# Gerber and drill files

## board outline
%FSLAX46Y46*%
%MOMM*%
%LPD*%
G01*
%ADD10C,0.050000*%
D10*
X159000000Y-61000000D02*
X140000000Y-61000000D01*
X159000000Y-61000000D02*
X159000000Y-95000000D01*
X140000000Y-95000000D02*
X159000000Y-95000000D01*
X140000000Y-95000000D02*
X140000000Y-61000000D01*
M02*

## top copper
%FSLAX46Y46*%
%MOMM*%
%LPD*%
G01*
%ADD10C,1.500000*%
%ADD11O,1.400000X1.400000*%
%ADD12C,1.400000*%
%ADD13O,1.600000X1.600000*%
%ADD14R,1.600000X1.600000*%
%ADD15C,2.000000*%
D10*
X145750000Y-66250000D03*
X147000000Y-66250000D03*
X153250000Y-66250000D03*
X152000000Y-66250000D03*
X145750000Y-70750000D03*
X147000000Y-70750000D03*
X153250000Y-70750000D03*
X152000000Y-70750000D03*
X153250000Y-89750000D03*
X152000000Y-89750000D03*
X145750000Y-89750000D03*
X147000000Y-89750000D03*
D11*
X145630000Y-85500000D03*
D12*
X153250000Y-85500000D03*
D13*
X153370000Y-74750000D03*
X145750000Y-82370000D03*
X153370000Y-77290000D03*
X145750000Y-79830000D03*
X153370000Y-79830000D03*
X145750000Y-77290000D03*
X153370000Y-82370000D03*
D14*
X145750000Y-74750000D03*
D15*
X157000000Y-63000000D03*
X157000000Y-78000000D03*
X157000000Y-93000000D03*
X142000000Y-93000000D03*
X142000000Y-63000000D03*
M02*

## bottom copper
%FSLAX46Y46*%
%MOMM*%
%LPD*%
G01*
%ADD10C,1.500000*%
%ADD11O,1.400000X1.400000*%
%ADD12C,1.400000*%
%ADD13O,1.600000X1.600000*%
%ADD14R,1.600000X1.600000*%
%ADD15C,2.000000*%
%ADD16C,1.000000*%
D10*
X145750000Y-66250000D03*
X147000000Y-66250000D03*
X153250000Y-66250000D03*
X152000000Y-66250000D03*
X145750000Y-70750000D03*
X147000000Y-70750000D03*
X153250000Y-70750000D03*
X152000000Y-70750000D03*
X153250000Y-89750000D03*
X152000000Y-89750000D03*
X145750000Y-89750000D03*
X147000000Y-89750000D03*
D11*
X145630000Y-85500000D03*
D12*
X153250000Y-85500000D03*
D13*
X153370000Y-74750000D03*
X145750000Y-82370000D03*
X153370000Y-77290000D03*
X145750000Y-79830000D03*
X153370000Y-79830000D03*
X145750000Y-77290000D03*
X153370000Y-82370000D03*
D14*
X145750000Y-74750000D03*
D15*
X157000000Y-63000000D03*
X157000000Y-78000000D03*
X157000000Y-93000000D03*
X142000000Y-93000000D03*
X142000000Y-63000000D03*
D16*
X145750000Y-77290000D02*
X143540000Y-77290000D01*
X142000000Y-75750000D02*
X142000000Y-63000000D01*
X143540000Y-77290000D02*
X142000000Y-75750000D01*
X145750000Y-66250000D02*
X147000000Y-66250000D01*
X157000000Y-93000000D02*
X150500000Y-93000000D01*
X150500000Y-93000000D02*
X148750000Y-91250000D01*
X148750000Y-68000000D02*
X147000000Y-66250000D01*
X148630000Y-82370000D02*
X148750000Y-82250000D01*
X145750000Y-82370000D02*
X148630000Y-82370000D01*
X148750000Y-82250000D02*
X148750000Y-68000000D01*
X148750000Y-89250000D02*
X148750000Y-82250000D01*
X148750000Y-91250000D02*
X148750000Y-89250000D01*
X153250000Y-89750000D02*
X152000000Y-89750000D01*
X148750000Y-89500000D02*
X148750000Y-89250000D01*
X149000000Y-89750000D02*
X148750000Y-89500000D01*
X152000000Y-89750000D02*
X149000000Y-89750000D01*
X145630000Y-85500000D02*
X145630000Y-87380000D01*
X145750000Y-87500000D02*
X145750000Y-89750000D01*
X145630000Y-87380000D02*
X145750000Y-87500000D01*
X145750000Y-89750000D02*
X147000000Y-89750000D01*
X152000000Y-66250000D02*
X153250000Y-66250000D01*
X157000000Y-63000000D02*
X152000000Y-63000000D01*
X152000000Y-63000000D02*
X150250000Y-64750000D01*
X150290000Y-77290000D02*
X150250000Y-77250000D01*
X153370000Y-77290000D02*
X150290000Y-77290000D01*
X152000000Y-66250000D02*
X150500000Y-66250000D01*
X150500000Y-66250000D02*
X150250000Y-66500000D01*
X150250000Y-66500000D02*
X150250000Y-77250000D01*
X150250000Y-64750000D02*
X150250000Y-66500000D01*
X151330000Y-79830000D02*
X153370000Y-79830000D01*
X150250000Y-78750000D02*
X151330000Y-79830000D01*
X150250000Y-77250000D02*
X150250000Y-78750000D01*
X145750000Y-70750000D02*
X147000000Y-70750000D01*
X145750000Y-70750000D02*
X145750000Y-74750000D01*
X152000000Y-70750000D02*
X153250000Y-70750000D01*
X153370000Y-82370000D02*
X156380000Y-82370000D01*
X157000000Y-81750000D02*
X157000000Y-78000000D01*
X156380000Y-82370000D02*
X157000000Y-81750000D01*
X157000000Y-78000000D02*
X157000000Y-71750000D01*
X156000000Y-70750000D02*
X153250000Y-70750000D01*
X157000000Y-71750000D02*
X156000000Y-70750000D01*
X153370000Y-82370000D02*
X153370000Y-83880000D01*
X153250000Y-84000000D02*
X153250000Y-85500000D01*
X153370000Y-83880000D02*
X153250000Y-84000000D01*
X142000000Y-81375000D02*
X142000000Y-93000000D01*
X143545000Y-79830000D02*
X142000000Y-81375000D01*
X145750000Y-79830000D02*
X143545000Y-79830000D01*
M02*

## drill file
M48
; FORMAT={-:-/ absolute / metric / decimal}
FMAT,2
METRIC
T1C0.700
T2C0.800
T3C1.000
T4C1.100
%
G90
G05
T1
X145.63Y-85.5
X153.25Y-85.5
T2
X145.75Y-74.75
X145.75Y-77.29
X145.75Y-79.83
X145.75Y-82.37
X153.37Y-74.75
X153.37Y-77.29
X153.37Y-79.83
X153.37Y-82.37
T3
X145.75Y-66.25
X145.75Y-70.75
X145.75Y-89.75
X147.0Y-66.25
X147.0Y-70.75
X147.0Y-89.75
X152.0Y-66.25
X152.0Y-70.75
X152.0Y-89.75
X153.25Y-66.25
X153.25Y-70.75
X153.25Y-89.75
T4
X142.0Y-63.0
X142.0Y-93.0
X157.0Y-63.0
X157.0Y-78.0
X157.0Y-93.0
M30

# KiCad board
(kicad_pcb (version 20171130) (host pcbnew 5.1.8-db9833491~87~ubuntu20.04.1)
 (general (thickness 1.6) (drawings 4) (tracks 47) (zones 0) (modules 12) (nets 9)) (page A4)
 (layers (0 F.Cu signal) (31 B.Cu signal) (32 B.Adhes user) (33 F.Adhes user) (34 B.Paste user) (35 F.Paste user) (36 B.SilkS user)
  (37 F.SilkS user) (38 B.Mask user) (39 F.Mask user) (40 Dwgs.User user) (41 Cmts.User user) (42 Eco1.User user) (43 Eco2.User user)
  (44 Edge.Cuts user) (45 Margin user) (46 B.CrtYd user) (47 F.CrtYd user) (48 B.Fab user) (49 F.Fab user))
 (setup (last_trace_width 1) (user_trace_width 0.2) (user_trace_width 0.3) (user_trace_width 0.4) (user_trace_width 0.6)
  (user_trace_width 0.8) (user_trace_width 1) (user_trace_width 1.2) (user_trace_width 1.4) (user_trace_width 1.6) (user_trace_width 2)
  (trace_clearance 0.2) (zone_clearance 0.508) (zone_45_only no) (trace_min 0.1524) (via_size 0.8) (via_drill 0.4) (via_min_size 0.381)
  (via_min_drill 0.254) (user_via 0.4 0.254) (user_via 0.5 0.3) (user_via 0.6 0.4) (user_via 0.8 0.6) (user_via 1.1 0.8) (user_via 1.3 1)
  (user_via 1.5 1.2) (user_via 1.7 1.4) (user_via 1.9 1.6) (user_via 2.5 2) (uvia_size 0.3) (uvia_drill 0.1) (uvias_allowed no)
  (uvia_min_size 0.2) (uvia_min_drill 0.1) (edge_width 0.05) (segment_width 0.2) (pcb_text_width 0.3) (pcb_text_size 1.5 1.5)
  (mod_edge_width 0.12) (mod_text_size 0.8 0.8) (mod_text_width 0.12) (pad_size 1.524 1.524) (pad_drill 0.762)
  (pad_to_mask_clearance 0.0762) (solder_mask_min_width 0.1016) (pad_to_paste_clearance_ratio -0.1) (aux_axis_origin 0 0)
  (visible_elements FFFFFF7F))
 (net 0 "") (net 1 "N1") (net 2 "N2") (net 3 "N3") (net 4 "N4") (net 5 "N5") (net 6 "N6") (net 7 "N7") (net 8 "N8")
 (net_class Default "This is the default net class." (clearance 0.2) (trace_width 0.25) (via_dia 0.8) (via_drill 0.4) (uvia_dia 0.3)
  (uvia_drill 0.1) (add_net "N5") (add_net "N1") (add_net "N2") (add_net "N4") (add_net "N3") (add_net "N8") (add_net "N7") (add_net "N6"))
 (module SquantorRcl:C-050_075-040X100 (layer F.Cu) (at 149.5 66.25 180)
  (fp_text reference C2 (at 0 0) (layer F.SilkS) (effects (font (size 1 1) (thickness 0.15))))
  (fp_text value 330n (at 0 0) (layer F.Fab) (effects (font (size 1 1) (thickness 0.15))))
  (pad 2 thru_hole circle (at 3.75 0 180) (size 1.5 1.5) (drill 1) (layers *.Cu *.Mask) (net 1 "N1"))
  (pad 2 thru_hole circle (at 2.5 0 180) (size 1.5 1.5) (drill 1) (layers *.Cu *.Mask) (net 1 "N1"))
  (pad 1 thru_hole circle (at -3.75 0 180) (size 1.5 1.5) (drill 1) (layers *.Cu *.Mask) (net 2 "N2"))
  (pad 1 thru_hole circle (at -2.5 0 180) (size 1.5 1.5) (drill 1) (layers *.Cu *.Mask) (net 2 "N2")))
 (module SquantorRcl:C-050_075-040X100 (layer F.Cu) (at 149.5 70.75 180)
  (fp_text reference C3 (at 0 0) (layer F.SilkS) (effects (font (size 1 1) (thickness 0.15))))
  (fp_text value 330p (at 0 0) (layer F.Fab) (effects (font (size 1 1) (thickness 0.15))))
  (pad 2 thru_hole circle (at 3.75 0 180) (size 1.5 1.5) (drill 1) (layers *.Cu *.Mask) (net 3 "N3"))
  (pad 2 thru_hole circle (at 2.5 0 180) (size 1.5 1.5) (drill 1) (layers *.Cu *.Mask) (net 3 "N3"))
  (pad 1 thru_hole circle (at -3.75 0 180) (size 1.5 1.5) (drill 1) (layers *.Cu *.Mask) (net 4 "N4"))
  (pad 1 thru_hole circle (at -2.5 0 180) (size 1.5 1.5) (drill 1) (layers *.Cu *.Mask) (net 4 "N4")))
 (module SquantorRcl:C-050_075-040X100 (layer F.Cu) (at 149.5 89.75)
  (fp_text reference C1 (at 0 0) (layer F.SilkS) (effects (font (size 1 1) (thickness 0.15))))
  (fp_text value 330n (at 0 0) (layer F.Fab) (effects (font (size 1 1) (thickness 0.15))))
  (pad 2 thru_hole circle (at 3.75 0) (size 1.5 1.5) (drill 1) (layers *.Cu *.Mask) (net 1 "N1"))
  (pad 2 thru_hole circle (at 2.5 0) (size 1.5 1.5) (drill 1) (layers *.Cu *.Mask) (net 1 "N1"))
  (pad 1 thru_hole circle (at -3.75 0) (size 1.5 1.5) (drill 1) (layers *.Cu *.Mask) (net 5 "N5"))
  (pad 1 thru_hole circle (at -2.5 0) (size 1.5 1.5) (drill 1) (layers *.Cu *.Mask) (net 5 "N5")))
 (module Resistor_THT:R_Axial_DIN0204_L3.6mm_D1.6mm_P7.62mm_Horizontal (layer F.Cu) (at 153.25 85.5 180)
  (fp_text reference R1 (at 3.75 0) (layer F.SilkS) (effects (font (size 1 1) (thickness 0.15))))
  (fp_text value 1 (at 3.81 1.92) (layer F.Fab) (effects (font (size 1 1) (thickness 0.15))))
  (pad 2 thru_hole oval (at 7.62 0 180) (size 1.4 1.4) (drill 0.7) (layers *.Cu *.Mask) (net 5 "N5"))
  (pad 1 thru_hole circle (at 0 0 180) (size 1.4 1.4) (drill 0.7) (layers *.Cu *.Mask) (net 4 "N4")))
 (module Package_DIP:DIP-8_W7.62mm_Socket (layer F.Cu) (at 145.75 74.75)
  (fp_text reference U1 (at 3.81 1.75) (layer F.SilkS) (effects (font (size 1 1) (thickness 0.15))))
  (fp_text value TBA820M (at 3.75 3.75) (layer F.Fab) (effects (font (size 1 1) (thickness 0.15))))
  (pad 8 thru_hole oval (at 7.62 0) (size 1.6 1.6) (drill 0.8) (layers *.Cu *.Mask) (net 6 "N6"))
  (pad 4 thru_hole oval (at 0 7.62) (size 1.6 1.6) (drill 0.8) (layers *.Cu *.Mask) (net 1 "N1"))
  (pad 7 thru_hole oval (at 7.62 2.54) (size 1.6 1.6) (drill 0.8) (layers *.Cu *.Mask) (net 2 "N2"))
  (pad 3 thru_hole oval (at 0 5.08) (size 1.6 1.6) (drill 0.8) (layers *.Cu *.Mask) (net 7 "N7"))
  (pad 6 thru_hole oval (at 7.62 5.08) (size 1.6 1.6) (drill 0.8) (layers *.Cu *.Mask) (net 2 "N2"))
  (pad 2 thru_hole oval (at 0 2.54) (size 1.6 1.6) (drill 0.8) (layers *.Cu *.Mask) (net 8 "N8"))
  (pad 5 thru_hole oval (at 7.62 7.62) (size 1.6 1.6) (drill 0.8) (layers *.Cu *.Mask) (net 4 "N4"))
  (pad 1 thru_hole rect (at 0 0) (size 1.6 1.6) (drill 0.8) (layers *.Cu *.Mask) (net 3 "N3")))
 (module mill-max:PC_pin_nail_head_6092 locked (layer F.Cu) (at 157 63)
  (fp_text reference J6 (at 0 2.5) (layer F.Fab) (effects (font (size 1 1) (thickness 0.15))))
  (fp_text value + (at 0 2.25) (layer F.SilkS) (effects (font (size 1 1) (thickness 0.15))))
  (pad 1 thru_hole circle (at 0 0) (size 2 2) (drill 1.1) (layers *.Cu *.Mask) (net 2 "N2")))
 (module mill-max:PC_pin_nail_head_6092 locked (layer F.Cu) (at 157 78)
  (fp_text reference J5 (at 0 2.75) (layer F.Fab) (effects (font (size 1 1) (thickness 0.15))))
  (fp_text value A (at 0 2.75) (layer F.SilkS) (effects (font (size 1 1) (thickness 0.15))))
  (pad 1 thru_hole circle (at 0 0) (size 2 2) (drill 1.1) (layers *.Cu *.Mask) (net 4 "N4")))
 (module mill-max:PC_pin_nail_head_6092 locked (layer F.Cu) (at 157 93)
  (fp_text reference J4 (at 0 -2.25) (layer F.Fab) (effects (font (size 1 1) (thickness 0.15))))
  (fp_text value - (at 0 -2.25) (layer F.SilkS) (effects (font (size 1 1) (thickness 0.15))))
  (pad 1 thru_hole circle (at 0 0) (size 2 2) (drill 1.1) (layers *.Cu *.Mask) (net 1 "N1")))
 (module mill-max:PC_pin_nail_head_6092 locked (layer F.Cu) (at 142 93)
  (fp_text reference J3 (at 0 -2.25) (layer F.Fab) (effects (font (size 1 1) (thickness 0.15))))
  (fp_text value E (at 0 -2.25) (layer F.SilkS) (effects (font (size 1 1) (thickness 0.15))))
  (pad 1 thru_hole circle (at 0 0) (size 2 2) (drill 1.1) (layers *.Cu *.Mask) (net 7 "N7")))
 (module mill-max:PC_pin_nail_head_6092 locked (layer F.Cu) (at 142 63)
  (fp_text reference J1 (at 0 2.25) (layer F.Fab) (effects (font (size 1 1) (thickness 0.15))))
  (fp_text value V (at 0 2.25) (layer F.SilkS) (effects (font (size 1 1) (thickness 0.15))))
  (pad 1 thru_hole circle (at 0 0) (size 2 2) (drill 1.1) (layers *.Cu *.Mask) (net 8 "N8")))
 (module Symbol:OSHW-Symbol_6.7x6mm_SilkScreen (layer B.Cu) (at 149.5 83.75 180)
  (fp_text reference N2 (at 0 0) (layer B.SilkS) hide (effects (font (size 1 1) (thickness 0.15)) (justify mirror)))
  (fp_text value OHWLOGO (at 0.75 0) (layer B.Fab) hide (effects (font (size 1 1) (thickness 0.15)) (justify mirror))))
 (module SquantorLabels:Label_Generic (layer B.Cu) (at 148.5 87.5)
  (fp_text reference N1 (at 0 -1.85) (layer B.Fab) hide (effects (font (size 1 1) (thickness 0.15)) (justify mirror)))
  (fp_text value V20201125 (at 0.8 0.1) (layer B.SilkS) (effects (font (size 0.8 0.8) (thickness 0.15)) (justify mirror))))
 (gr_line (start 159 61) (end 140 61) (layer Edge.Cuts) (width 0.05))
 (gr_line (start 159 61) (end 159 95) (layer Edge.Cuts) (width 0.05))
 (gr_line (start 140 95) (end 159 95) (layer Edge.Cuts) (width 0.05))
 (gr_line (start 140 95) (end 140 61) (layer Edge.Cuts) (width 0.05))
 (segment (start 145.75 77.29) (end 143.54 77.29) (width 1) (layer B.Cu) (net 8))
 (segment (start 142 75.75) (end 142 63) (width 1) (layer B.Cu) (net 8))
 (segment (start 143.54 77.29) (end 142 75.75) (width 1) (layer B.Cu) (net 8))
 (segment (start 145.75 66.25) (end 147 66.25) (width 1) (layer B.Cu) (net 1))
 (segment (start 157 93) (end 150.5 93) (width 1) (layer B.Cu) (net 1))
 (segment (start 150.5 93) (end 148.75 91.25) (width 1) (layer B.Cu) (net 1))
 (segment (start 148.75 68) (end 147 66.25) (width 1) (layer B.Cu) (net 1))
 (segment (start 148.63 82.37) (end 148.75 82.25) (width 1) (layer B.Cu) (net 1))
 (segment (start 145.75 82.37) (end 148.63 82.37) (width 1) (layer B.Cu) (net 1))
 (segment (start 148.75 82.25) (end 148.75 68) (width 1) (layer B.Cu) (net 1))
 (segment (start 148.75 89.25) (end 148.75 82.25) (width 1) (layer B.Cu) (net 1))
 (segment (start 148.75 91.25) (end 148.75 89.25) (width 1) (layer B.Cu) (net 1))
 (segment (start 153.25 89.75) (end 152 89.75) (width 1) (layer B.Cu) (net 1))
 (segment (start 148.75 89.5) (end 148.75 89.25) (width 1) (layer B.Cu) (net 1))
 (segment (start 149 89.75) (end 148.75 89.5) (width 1) (layer B.Cu) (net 1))
 (segment (start 152 89.75) (end 149 89.75) (width 1) (layer B.Cu) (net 1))
 (segment (start 145.63 85.5) (end 145.63 87.38) (width 1) (layer B.Cu) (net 5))
 (segment (start 145.75 87.5) (end 145.75 89.75) (width 1) (layer B.Cu) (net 5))
 (segment (start 145.63 87.38) (end 145.75 87.5) (width 1) (layer B.Cu) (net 5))
 (segment (start 145.75 89.75) (end 147 89.75) (width 1) (layer B.Cu) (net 5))
 (segment (start 152 66.25) (end 153.25 66.25) (width 1) (layer B.Cu) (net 2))
 (segment (start 157 63) (end 152 63) (width 1) (layer B.Cu) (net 2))
 (segment (start 152 63) (end 150.25 64.75) (width 1) (layer B.Cu) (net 2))
 (segment (start 150.29 77.29) (end 150.25 77.25) (width 1) (layer B.Cu) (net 2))
 (segment (start 153.37 77.29) (end 150.29 77.29) (width 1) (layer B.Cu) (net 2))
 (segment (start 152 66.25) (end 150.5 66.25) (width 1) (layer B.Cu) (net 2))
 (segment (start 150.5 66.25) (end 150.25 66.5) (width 1) (layer B.Cu) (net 2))
 (segment (start 150.25 66.5) (end 150.25 77.25) (width 1) (layer B.Cu) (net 2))
 (segment (start 150.25 64.75) (end 150.25 66.5) (width 1) (layer B.Cu) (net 2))
 (segment (start 151.33 79.83) (end 153.37 79.83) (width 1) (layer B.Cu) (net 2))
 (segment (start 150.25 78.75) (end 151.33 79.83) (width 1) (layer B.Cu) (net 2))
 (segment (start 150.25 77.25) (end 150.25 78.75) (width 1) (layer B.Cu) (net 2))
 (segment (start 145.75 70.75) (end 147 70.75) (width 1) (layer B.Cu) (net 3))
 (segment (start 145.75 70.75) (end 145.75 74.75) (width 1) (layer B.Cu) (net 3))
 (segment (start 152 70.75) (end 153.25 70.75) (width 1) (layer B.Cu) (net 4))
 (segment (start 153.37 82.37) (end 156.38 82.37) (width 1) (layer B.Cu) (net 4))
 (segment (start 157 81.75) (end 157 78) (width 1) (layer B.Cu) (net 4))
 (segment (start 156.38 82.37) (end 157 81.75) (width 1) (layer B.Cu) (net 4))
 (segment (start 157 78) (end 157 71.75) (width 1) (layer B.Cu) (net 4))
 (segment (start 156 70.75) (end 153.25 70.75) (width 1) (layer B.Cu) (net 4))
 (segment (start 157 71.75) (end 156 70.75) (width 1) (layer B.Cu) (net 4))
 (segment (start 153.37 82.37) (end 153.37 83.88) (width 1) (layer B.Cu) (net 4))
 (segment (start 153.25 84) (end 153.25 85.5) (width 1) (layer B.Cu) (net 4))
 (segment (start 153.37 83.88) (end 153.25 84) (width 1) (layer B.Cu) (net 4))
 (segment (start 142 81.375) (end 142 93) (width 1) (layer B.Cu) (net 7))
 (segment (start 143.545 79.83) (end 142 81.375) (width 1) (layer B.Cu) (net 7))
 (segment (start 145.75 79.83) (end 143.545 79.83) (width 1) (layer B.Cu) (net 7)))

